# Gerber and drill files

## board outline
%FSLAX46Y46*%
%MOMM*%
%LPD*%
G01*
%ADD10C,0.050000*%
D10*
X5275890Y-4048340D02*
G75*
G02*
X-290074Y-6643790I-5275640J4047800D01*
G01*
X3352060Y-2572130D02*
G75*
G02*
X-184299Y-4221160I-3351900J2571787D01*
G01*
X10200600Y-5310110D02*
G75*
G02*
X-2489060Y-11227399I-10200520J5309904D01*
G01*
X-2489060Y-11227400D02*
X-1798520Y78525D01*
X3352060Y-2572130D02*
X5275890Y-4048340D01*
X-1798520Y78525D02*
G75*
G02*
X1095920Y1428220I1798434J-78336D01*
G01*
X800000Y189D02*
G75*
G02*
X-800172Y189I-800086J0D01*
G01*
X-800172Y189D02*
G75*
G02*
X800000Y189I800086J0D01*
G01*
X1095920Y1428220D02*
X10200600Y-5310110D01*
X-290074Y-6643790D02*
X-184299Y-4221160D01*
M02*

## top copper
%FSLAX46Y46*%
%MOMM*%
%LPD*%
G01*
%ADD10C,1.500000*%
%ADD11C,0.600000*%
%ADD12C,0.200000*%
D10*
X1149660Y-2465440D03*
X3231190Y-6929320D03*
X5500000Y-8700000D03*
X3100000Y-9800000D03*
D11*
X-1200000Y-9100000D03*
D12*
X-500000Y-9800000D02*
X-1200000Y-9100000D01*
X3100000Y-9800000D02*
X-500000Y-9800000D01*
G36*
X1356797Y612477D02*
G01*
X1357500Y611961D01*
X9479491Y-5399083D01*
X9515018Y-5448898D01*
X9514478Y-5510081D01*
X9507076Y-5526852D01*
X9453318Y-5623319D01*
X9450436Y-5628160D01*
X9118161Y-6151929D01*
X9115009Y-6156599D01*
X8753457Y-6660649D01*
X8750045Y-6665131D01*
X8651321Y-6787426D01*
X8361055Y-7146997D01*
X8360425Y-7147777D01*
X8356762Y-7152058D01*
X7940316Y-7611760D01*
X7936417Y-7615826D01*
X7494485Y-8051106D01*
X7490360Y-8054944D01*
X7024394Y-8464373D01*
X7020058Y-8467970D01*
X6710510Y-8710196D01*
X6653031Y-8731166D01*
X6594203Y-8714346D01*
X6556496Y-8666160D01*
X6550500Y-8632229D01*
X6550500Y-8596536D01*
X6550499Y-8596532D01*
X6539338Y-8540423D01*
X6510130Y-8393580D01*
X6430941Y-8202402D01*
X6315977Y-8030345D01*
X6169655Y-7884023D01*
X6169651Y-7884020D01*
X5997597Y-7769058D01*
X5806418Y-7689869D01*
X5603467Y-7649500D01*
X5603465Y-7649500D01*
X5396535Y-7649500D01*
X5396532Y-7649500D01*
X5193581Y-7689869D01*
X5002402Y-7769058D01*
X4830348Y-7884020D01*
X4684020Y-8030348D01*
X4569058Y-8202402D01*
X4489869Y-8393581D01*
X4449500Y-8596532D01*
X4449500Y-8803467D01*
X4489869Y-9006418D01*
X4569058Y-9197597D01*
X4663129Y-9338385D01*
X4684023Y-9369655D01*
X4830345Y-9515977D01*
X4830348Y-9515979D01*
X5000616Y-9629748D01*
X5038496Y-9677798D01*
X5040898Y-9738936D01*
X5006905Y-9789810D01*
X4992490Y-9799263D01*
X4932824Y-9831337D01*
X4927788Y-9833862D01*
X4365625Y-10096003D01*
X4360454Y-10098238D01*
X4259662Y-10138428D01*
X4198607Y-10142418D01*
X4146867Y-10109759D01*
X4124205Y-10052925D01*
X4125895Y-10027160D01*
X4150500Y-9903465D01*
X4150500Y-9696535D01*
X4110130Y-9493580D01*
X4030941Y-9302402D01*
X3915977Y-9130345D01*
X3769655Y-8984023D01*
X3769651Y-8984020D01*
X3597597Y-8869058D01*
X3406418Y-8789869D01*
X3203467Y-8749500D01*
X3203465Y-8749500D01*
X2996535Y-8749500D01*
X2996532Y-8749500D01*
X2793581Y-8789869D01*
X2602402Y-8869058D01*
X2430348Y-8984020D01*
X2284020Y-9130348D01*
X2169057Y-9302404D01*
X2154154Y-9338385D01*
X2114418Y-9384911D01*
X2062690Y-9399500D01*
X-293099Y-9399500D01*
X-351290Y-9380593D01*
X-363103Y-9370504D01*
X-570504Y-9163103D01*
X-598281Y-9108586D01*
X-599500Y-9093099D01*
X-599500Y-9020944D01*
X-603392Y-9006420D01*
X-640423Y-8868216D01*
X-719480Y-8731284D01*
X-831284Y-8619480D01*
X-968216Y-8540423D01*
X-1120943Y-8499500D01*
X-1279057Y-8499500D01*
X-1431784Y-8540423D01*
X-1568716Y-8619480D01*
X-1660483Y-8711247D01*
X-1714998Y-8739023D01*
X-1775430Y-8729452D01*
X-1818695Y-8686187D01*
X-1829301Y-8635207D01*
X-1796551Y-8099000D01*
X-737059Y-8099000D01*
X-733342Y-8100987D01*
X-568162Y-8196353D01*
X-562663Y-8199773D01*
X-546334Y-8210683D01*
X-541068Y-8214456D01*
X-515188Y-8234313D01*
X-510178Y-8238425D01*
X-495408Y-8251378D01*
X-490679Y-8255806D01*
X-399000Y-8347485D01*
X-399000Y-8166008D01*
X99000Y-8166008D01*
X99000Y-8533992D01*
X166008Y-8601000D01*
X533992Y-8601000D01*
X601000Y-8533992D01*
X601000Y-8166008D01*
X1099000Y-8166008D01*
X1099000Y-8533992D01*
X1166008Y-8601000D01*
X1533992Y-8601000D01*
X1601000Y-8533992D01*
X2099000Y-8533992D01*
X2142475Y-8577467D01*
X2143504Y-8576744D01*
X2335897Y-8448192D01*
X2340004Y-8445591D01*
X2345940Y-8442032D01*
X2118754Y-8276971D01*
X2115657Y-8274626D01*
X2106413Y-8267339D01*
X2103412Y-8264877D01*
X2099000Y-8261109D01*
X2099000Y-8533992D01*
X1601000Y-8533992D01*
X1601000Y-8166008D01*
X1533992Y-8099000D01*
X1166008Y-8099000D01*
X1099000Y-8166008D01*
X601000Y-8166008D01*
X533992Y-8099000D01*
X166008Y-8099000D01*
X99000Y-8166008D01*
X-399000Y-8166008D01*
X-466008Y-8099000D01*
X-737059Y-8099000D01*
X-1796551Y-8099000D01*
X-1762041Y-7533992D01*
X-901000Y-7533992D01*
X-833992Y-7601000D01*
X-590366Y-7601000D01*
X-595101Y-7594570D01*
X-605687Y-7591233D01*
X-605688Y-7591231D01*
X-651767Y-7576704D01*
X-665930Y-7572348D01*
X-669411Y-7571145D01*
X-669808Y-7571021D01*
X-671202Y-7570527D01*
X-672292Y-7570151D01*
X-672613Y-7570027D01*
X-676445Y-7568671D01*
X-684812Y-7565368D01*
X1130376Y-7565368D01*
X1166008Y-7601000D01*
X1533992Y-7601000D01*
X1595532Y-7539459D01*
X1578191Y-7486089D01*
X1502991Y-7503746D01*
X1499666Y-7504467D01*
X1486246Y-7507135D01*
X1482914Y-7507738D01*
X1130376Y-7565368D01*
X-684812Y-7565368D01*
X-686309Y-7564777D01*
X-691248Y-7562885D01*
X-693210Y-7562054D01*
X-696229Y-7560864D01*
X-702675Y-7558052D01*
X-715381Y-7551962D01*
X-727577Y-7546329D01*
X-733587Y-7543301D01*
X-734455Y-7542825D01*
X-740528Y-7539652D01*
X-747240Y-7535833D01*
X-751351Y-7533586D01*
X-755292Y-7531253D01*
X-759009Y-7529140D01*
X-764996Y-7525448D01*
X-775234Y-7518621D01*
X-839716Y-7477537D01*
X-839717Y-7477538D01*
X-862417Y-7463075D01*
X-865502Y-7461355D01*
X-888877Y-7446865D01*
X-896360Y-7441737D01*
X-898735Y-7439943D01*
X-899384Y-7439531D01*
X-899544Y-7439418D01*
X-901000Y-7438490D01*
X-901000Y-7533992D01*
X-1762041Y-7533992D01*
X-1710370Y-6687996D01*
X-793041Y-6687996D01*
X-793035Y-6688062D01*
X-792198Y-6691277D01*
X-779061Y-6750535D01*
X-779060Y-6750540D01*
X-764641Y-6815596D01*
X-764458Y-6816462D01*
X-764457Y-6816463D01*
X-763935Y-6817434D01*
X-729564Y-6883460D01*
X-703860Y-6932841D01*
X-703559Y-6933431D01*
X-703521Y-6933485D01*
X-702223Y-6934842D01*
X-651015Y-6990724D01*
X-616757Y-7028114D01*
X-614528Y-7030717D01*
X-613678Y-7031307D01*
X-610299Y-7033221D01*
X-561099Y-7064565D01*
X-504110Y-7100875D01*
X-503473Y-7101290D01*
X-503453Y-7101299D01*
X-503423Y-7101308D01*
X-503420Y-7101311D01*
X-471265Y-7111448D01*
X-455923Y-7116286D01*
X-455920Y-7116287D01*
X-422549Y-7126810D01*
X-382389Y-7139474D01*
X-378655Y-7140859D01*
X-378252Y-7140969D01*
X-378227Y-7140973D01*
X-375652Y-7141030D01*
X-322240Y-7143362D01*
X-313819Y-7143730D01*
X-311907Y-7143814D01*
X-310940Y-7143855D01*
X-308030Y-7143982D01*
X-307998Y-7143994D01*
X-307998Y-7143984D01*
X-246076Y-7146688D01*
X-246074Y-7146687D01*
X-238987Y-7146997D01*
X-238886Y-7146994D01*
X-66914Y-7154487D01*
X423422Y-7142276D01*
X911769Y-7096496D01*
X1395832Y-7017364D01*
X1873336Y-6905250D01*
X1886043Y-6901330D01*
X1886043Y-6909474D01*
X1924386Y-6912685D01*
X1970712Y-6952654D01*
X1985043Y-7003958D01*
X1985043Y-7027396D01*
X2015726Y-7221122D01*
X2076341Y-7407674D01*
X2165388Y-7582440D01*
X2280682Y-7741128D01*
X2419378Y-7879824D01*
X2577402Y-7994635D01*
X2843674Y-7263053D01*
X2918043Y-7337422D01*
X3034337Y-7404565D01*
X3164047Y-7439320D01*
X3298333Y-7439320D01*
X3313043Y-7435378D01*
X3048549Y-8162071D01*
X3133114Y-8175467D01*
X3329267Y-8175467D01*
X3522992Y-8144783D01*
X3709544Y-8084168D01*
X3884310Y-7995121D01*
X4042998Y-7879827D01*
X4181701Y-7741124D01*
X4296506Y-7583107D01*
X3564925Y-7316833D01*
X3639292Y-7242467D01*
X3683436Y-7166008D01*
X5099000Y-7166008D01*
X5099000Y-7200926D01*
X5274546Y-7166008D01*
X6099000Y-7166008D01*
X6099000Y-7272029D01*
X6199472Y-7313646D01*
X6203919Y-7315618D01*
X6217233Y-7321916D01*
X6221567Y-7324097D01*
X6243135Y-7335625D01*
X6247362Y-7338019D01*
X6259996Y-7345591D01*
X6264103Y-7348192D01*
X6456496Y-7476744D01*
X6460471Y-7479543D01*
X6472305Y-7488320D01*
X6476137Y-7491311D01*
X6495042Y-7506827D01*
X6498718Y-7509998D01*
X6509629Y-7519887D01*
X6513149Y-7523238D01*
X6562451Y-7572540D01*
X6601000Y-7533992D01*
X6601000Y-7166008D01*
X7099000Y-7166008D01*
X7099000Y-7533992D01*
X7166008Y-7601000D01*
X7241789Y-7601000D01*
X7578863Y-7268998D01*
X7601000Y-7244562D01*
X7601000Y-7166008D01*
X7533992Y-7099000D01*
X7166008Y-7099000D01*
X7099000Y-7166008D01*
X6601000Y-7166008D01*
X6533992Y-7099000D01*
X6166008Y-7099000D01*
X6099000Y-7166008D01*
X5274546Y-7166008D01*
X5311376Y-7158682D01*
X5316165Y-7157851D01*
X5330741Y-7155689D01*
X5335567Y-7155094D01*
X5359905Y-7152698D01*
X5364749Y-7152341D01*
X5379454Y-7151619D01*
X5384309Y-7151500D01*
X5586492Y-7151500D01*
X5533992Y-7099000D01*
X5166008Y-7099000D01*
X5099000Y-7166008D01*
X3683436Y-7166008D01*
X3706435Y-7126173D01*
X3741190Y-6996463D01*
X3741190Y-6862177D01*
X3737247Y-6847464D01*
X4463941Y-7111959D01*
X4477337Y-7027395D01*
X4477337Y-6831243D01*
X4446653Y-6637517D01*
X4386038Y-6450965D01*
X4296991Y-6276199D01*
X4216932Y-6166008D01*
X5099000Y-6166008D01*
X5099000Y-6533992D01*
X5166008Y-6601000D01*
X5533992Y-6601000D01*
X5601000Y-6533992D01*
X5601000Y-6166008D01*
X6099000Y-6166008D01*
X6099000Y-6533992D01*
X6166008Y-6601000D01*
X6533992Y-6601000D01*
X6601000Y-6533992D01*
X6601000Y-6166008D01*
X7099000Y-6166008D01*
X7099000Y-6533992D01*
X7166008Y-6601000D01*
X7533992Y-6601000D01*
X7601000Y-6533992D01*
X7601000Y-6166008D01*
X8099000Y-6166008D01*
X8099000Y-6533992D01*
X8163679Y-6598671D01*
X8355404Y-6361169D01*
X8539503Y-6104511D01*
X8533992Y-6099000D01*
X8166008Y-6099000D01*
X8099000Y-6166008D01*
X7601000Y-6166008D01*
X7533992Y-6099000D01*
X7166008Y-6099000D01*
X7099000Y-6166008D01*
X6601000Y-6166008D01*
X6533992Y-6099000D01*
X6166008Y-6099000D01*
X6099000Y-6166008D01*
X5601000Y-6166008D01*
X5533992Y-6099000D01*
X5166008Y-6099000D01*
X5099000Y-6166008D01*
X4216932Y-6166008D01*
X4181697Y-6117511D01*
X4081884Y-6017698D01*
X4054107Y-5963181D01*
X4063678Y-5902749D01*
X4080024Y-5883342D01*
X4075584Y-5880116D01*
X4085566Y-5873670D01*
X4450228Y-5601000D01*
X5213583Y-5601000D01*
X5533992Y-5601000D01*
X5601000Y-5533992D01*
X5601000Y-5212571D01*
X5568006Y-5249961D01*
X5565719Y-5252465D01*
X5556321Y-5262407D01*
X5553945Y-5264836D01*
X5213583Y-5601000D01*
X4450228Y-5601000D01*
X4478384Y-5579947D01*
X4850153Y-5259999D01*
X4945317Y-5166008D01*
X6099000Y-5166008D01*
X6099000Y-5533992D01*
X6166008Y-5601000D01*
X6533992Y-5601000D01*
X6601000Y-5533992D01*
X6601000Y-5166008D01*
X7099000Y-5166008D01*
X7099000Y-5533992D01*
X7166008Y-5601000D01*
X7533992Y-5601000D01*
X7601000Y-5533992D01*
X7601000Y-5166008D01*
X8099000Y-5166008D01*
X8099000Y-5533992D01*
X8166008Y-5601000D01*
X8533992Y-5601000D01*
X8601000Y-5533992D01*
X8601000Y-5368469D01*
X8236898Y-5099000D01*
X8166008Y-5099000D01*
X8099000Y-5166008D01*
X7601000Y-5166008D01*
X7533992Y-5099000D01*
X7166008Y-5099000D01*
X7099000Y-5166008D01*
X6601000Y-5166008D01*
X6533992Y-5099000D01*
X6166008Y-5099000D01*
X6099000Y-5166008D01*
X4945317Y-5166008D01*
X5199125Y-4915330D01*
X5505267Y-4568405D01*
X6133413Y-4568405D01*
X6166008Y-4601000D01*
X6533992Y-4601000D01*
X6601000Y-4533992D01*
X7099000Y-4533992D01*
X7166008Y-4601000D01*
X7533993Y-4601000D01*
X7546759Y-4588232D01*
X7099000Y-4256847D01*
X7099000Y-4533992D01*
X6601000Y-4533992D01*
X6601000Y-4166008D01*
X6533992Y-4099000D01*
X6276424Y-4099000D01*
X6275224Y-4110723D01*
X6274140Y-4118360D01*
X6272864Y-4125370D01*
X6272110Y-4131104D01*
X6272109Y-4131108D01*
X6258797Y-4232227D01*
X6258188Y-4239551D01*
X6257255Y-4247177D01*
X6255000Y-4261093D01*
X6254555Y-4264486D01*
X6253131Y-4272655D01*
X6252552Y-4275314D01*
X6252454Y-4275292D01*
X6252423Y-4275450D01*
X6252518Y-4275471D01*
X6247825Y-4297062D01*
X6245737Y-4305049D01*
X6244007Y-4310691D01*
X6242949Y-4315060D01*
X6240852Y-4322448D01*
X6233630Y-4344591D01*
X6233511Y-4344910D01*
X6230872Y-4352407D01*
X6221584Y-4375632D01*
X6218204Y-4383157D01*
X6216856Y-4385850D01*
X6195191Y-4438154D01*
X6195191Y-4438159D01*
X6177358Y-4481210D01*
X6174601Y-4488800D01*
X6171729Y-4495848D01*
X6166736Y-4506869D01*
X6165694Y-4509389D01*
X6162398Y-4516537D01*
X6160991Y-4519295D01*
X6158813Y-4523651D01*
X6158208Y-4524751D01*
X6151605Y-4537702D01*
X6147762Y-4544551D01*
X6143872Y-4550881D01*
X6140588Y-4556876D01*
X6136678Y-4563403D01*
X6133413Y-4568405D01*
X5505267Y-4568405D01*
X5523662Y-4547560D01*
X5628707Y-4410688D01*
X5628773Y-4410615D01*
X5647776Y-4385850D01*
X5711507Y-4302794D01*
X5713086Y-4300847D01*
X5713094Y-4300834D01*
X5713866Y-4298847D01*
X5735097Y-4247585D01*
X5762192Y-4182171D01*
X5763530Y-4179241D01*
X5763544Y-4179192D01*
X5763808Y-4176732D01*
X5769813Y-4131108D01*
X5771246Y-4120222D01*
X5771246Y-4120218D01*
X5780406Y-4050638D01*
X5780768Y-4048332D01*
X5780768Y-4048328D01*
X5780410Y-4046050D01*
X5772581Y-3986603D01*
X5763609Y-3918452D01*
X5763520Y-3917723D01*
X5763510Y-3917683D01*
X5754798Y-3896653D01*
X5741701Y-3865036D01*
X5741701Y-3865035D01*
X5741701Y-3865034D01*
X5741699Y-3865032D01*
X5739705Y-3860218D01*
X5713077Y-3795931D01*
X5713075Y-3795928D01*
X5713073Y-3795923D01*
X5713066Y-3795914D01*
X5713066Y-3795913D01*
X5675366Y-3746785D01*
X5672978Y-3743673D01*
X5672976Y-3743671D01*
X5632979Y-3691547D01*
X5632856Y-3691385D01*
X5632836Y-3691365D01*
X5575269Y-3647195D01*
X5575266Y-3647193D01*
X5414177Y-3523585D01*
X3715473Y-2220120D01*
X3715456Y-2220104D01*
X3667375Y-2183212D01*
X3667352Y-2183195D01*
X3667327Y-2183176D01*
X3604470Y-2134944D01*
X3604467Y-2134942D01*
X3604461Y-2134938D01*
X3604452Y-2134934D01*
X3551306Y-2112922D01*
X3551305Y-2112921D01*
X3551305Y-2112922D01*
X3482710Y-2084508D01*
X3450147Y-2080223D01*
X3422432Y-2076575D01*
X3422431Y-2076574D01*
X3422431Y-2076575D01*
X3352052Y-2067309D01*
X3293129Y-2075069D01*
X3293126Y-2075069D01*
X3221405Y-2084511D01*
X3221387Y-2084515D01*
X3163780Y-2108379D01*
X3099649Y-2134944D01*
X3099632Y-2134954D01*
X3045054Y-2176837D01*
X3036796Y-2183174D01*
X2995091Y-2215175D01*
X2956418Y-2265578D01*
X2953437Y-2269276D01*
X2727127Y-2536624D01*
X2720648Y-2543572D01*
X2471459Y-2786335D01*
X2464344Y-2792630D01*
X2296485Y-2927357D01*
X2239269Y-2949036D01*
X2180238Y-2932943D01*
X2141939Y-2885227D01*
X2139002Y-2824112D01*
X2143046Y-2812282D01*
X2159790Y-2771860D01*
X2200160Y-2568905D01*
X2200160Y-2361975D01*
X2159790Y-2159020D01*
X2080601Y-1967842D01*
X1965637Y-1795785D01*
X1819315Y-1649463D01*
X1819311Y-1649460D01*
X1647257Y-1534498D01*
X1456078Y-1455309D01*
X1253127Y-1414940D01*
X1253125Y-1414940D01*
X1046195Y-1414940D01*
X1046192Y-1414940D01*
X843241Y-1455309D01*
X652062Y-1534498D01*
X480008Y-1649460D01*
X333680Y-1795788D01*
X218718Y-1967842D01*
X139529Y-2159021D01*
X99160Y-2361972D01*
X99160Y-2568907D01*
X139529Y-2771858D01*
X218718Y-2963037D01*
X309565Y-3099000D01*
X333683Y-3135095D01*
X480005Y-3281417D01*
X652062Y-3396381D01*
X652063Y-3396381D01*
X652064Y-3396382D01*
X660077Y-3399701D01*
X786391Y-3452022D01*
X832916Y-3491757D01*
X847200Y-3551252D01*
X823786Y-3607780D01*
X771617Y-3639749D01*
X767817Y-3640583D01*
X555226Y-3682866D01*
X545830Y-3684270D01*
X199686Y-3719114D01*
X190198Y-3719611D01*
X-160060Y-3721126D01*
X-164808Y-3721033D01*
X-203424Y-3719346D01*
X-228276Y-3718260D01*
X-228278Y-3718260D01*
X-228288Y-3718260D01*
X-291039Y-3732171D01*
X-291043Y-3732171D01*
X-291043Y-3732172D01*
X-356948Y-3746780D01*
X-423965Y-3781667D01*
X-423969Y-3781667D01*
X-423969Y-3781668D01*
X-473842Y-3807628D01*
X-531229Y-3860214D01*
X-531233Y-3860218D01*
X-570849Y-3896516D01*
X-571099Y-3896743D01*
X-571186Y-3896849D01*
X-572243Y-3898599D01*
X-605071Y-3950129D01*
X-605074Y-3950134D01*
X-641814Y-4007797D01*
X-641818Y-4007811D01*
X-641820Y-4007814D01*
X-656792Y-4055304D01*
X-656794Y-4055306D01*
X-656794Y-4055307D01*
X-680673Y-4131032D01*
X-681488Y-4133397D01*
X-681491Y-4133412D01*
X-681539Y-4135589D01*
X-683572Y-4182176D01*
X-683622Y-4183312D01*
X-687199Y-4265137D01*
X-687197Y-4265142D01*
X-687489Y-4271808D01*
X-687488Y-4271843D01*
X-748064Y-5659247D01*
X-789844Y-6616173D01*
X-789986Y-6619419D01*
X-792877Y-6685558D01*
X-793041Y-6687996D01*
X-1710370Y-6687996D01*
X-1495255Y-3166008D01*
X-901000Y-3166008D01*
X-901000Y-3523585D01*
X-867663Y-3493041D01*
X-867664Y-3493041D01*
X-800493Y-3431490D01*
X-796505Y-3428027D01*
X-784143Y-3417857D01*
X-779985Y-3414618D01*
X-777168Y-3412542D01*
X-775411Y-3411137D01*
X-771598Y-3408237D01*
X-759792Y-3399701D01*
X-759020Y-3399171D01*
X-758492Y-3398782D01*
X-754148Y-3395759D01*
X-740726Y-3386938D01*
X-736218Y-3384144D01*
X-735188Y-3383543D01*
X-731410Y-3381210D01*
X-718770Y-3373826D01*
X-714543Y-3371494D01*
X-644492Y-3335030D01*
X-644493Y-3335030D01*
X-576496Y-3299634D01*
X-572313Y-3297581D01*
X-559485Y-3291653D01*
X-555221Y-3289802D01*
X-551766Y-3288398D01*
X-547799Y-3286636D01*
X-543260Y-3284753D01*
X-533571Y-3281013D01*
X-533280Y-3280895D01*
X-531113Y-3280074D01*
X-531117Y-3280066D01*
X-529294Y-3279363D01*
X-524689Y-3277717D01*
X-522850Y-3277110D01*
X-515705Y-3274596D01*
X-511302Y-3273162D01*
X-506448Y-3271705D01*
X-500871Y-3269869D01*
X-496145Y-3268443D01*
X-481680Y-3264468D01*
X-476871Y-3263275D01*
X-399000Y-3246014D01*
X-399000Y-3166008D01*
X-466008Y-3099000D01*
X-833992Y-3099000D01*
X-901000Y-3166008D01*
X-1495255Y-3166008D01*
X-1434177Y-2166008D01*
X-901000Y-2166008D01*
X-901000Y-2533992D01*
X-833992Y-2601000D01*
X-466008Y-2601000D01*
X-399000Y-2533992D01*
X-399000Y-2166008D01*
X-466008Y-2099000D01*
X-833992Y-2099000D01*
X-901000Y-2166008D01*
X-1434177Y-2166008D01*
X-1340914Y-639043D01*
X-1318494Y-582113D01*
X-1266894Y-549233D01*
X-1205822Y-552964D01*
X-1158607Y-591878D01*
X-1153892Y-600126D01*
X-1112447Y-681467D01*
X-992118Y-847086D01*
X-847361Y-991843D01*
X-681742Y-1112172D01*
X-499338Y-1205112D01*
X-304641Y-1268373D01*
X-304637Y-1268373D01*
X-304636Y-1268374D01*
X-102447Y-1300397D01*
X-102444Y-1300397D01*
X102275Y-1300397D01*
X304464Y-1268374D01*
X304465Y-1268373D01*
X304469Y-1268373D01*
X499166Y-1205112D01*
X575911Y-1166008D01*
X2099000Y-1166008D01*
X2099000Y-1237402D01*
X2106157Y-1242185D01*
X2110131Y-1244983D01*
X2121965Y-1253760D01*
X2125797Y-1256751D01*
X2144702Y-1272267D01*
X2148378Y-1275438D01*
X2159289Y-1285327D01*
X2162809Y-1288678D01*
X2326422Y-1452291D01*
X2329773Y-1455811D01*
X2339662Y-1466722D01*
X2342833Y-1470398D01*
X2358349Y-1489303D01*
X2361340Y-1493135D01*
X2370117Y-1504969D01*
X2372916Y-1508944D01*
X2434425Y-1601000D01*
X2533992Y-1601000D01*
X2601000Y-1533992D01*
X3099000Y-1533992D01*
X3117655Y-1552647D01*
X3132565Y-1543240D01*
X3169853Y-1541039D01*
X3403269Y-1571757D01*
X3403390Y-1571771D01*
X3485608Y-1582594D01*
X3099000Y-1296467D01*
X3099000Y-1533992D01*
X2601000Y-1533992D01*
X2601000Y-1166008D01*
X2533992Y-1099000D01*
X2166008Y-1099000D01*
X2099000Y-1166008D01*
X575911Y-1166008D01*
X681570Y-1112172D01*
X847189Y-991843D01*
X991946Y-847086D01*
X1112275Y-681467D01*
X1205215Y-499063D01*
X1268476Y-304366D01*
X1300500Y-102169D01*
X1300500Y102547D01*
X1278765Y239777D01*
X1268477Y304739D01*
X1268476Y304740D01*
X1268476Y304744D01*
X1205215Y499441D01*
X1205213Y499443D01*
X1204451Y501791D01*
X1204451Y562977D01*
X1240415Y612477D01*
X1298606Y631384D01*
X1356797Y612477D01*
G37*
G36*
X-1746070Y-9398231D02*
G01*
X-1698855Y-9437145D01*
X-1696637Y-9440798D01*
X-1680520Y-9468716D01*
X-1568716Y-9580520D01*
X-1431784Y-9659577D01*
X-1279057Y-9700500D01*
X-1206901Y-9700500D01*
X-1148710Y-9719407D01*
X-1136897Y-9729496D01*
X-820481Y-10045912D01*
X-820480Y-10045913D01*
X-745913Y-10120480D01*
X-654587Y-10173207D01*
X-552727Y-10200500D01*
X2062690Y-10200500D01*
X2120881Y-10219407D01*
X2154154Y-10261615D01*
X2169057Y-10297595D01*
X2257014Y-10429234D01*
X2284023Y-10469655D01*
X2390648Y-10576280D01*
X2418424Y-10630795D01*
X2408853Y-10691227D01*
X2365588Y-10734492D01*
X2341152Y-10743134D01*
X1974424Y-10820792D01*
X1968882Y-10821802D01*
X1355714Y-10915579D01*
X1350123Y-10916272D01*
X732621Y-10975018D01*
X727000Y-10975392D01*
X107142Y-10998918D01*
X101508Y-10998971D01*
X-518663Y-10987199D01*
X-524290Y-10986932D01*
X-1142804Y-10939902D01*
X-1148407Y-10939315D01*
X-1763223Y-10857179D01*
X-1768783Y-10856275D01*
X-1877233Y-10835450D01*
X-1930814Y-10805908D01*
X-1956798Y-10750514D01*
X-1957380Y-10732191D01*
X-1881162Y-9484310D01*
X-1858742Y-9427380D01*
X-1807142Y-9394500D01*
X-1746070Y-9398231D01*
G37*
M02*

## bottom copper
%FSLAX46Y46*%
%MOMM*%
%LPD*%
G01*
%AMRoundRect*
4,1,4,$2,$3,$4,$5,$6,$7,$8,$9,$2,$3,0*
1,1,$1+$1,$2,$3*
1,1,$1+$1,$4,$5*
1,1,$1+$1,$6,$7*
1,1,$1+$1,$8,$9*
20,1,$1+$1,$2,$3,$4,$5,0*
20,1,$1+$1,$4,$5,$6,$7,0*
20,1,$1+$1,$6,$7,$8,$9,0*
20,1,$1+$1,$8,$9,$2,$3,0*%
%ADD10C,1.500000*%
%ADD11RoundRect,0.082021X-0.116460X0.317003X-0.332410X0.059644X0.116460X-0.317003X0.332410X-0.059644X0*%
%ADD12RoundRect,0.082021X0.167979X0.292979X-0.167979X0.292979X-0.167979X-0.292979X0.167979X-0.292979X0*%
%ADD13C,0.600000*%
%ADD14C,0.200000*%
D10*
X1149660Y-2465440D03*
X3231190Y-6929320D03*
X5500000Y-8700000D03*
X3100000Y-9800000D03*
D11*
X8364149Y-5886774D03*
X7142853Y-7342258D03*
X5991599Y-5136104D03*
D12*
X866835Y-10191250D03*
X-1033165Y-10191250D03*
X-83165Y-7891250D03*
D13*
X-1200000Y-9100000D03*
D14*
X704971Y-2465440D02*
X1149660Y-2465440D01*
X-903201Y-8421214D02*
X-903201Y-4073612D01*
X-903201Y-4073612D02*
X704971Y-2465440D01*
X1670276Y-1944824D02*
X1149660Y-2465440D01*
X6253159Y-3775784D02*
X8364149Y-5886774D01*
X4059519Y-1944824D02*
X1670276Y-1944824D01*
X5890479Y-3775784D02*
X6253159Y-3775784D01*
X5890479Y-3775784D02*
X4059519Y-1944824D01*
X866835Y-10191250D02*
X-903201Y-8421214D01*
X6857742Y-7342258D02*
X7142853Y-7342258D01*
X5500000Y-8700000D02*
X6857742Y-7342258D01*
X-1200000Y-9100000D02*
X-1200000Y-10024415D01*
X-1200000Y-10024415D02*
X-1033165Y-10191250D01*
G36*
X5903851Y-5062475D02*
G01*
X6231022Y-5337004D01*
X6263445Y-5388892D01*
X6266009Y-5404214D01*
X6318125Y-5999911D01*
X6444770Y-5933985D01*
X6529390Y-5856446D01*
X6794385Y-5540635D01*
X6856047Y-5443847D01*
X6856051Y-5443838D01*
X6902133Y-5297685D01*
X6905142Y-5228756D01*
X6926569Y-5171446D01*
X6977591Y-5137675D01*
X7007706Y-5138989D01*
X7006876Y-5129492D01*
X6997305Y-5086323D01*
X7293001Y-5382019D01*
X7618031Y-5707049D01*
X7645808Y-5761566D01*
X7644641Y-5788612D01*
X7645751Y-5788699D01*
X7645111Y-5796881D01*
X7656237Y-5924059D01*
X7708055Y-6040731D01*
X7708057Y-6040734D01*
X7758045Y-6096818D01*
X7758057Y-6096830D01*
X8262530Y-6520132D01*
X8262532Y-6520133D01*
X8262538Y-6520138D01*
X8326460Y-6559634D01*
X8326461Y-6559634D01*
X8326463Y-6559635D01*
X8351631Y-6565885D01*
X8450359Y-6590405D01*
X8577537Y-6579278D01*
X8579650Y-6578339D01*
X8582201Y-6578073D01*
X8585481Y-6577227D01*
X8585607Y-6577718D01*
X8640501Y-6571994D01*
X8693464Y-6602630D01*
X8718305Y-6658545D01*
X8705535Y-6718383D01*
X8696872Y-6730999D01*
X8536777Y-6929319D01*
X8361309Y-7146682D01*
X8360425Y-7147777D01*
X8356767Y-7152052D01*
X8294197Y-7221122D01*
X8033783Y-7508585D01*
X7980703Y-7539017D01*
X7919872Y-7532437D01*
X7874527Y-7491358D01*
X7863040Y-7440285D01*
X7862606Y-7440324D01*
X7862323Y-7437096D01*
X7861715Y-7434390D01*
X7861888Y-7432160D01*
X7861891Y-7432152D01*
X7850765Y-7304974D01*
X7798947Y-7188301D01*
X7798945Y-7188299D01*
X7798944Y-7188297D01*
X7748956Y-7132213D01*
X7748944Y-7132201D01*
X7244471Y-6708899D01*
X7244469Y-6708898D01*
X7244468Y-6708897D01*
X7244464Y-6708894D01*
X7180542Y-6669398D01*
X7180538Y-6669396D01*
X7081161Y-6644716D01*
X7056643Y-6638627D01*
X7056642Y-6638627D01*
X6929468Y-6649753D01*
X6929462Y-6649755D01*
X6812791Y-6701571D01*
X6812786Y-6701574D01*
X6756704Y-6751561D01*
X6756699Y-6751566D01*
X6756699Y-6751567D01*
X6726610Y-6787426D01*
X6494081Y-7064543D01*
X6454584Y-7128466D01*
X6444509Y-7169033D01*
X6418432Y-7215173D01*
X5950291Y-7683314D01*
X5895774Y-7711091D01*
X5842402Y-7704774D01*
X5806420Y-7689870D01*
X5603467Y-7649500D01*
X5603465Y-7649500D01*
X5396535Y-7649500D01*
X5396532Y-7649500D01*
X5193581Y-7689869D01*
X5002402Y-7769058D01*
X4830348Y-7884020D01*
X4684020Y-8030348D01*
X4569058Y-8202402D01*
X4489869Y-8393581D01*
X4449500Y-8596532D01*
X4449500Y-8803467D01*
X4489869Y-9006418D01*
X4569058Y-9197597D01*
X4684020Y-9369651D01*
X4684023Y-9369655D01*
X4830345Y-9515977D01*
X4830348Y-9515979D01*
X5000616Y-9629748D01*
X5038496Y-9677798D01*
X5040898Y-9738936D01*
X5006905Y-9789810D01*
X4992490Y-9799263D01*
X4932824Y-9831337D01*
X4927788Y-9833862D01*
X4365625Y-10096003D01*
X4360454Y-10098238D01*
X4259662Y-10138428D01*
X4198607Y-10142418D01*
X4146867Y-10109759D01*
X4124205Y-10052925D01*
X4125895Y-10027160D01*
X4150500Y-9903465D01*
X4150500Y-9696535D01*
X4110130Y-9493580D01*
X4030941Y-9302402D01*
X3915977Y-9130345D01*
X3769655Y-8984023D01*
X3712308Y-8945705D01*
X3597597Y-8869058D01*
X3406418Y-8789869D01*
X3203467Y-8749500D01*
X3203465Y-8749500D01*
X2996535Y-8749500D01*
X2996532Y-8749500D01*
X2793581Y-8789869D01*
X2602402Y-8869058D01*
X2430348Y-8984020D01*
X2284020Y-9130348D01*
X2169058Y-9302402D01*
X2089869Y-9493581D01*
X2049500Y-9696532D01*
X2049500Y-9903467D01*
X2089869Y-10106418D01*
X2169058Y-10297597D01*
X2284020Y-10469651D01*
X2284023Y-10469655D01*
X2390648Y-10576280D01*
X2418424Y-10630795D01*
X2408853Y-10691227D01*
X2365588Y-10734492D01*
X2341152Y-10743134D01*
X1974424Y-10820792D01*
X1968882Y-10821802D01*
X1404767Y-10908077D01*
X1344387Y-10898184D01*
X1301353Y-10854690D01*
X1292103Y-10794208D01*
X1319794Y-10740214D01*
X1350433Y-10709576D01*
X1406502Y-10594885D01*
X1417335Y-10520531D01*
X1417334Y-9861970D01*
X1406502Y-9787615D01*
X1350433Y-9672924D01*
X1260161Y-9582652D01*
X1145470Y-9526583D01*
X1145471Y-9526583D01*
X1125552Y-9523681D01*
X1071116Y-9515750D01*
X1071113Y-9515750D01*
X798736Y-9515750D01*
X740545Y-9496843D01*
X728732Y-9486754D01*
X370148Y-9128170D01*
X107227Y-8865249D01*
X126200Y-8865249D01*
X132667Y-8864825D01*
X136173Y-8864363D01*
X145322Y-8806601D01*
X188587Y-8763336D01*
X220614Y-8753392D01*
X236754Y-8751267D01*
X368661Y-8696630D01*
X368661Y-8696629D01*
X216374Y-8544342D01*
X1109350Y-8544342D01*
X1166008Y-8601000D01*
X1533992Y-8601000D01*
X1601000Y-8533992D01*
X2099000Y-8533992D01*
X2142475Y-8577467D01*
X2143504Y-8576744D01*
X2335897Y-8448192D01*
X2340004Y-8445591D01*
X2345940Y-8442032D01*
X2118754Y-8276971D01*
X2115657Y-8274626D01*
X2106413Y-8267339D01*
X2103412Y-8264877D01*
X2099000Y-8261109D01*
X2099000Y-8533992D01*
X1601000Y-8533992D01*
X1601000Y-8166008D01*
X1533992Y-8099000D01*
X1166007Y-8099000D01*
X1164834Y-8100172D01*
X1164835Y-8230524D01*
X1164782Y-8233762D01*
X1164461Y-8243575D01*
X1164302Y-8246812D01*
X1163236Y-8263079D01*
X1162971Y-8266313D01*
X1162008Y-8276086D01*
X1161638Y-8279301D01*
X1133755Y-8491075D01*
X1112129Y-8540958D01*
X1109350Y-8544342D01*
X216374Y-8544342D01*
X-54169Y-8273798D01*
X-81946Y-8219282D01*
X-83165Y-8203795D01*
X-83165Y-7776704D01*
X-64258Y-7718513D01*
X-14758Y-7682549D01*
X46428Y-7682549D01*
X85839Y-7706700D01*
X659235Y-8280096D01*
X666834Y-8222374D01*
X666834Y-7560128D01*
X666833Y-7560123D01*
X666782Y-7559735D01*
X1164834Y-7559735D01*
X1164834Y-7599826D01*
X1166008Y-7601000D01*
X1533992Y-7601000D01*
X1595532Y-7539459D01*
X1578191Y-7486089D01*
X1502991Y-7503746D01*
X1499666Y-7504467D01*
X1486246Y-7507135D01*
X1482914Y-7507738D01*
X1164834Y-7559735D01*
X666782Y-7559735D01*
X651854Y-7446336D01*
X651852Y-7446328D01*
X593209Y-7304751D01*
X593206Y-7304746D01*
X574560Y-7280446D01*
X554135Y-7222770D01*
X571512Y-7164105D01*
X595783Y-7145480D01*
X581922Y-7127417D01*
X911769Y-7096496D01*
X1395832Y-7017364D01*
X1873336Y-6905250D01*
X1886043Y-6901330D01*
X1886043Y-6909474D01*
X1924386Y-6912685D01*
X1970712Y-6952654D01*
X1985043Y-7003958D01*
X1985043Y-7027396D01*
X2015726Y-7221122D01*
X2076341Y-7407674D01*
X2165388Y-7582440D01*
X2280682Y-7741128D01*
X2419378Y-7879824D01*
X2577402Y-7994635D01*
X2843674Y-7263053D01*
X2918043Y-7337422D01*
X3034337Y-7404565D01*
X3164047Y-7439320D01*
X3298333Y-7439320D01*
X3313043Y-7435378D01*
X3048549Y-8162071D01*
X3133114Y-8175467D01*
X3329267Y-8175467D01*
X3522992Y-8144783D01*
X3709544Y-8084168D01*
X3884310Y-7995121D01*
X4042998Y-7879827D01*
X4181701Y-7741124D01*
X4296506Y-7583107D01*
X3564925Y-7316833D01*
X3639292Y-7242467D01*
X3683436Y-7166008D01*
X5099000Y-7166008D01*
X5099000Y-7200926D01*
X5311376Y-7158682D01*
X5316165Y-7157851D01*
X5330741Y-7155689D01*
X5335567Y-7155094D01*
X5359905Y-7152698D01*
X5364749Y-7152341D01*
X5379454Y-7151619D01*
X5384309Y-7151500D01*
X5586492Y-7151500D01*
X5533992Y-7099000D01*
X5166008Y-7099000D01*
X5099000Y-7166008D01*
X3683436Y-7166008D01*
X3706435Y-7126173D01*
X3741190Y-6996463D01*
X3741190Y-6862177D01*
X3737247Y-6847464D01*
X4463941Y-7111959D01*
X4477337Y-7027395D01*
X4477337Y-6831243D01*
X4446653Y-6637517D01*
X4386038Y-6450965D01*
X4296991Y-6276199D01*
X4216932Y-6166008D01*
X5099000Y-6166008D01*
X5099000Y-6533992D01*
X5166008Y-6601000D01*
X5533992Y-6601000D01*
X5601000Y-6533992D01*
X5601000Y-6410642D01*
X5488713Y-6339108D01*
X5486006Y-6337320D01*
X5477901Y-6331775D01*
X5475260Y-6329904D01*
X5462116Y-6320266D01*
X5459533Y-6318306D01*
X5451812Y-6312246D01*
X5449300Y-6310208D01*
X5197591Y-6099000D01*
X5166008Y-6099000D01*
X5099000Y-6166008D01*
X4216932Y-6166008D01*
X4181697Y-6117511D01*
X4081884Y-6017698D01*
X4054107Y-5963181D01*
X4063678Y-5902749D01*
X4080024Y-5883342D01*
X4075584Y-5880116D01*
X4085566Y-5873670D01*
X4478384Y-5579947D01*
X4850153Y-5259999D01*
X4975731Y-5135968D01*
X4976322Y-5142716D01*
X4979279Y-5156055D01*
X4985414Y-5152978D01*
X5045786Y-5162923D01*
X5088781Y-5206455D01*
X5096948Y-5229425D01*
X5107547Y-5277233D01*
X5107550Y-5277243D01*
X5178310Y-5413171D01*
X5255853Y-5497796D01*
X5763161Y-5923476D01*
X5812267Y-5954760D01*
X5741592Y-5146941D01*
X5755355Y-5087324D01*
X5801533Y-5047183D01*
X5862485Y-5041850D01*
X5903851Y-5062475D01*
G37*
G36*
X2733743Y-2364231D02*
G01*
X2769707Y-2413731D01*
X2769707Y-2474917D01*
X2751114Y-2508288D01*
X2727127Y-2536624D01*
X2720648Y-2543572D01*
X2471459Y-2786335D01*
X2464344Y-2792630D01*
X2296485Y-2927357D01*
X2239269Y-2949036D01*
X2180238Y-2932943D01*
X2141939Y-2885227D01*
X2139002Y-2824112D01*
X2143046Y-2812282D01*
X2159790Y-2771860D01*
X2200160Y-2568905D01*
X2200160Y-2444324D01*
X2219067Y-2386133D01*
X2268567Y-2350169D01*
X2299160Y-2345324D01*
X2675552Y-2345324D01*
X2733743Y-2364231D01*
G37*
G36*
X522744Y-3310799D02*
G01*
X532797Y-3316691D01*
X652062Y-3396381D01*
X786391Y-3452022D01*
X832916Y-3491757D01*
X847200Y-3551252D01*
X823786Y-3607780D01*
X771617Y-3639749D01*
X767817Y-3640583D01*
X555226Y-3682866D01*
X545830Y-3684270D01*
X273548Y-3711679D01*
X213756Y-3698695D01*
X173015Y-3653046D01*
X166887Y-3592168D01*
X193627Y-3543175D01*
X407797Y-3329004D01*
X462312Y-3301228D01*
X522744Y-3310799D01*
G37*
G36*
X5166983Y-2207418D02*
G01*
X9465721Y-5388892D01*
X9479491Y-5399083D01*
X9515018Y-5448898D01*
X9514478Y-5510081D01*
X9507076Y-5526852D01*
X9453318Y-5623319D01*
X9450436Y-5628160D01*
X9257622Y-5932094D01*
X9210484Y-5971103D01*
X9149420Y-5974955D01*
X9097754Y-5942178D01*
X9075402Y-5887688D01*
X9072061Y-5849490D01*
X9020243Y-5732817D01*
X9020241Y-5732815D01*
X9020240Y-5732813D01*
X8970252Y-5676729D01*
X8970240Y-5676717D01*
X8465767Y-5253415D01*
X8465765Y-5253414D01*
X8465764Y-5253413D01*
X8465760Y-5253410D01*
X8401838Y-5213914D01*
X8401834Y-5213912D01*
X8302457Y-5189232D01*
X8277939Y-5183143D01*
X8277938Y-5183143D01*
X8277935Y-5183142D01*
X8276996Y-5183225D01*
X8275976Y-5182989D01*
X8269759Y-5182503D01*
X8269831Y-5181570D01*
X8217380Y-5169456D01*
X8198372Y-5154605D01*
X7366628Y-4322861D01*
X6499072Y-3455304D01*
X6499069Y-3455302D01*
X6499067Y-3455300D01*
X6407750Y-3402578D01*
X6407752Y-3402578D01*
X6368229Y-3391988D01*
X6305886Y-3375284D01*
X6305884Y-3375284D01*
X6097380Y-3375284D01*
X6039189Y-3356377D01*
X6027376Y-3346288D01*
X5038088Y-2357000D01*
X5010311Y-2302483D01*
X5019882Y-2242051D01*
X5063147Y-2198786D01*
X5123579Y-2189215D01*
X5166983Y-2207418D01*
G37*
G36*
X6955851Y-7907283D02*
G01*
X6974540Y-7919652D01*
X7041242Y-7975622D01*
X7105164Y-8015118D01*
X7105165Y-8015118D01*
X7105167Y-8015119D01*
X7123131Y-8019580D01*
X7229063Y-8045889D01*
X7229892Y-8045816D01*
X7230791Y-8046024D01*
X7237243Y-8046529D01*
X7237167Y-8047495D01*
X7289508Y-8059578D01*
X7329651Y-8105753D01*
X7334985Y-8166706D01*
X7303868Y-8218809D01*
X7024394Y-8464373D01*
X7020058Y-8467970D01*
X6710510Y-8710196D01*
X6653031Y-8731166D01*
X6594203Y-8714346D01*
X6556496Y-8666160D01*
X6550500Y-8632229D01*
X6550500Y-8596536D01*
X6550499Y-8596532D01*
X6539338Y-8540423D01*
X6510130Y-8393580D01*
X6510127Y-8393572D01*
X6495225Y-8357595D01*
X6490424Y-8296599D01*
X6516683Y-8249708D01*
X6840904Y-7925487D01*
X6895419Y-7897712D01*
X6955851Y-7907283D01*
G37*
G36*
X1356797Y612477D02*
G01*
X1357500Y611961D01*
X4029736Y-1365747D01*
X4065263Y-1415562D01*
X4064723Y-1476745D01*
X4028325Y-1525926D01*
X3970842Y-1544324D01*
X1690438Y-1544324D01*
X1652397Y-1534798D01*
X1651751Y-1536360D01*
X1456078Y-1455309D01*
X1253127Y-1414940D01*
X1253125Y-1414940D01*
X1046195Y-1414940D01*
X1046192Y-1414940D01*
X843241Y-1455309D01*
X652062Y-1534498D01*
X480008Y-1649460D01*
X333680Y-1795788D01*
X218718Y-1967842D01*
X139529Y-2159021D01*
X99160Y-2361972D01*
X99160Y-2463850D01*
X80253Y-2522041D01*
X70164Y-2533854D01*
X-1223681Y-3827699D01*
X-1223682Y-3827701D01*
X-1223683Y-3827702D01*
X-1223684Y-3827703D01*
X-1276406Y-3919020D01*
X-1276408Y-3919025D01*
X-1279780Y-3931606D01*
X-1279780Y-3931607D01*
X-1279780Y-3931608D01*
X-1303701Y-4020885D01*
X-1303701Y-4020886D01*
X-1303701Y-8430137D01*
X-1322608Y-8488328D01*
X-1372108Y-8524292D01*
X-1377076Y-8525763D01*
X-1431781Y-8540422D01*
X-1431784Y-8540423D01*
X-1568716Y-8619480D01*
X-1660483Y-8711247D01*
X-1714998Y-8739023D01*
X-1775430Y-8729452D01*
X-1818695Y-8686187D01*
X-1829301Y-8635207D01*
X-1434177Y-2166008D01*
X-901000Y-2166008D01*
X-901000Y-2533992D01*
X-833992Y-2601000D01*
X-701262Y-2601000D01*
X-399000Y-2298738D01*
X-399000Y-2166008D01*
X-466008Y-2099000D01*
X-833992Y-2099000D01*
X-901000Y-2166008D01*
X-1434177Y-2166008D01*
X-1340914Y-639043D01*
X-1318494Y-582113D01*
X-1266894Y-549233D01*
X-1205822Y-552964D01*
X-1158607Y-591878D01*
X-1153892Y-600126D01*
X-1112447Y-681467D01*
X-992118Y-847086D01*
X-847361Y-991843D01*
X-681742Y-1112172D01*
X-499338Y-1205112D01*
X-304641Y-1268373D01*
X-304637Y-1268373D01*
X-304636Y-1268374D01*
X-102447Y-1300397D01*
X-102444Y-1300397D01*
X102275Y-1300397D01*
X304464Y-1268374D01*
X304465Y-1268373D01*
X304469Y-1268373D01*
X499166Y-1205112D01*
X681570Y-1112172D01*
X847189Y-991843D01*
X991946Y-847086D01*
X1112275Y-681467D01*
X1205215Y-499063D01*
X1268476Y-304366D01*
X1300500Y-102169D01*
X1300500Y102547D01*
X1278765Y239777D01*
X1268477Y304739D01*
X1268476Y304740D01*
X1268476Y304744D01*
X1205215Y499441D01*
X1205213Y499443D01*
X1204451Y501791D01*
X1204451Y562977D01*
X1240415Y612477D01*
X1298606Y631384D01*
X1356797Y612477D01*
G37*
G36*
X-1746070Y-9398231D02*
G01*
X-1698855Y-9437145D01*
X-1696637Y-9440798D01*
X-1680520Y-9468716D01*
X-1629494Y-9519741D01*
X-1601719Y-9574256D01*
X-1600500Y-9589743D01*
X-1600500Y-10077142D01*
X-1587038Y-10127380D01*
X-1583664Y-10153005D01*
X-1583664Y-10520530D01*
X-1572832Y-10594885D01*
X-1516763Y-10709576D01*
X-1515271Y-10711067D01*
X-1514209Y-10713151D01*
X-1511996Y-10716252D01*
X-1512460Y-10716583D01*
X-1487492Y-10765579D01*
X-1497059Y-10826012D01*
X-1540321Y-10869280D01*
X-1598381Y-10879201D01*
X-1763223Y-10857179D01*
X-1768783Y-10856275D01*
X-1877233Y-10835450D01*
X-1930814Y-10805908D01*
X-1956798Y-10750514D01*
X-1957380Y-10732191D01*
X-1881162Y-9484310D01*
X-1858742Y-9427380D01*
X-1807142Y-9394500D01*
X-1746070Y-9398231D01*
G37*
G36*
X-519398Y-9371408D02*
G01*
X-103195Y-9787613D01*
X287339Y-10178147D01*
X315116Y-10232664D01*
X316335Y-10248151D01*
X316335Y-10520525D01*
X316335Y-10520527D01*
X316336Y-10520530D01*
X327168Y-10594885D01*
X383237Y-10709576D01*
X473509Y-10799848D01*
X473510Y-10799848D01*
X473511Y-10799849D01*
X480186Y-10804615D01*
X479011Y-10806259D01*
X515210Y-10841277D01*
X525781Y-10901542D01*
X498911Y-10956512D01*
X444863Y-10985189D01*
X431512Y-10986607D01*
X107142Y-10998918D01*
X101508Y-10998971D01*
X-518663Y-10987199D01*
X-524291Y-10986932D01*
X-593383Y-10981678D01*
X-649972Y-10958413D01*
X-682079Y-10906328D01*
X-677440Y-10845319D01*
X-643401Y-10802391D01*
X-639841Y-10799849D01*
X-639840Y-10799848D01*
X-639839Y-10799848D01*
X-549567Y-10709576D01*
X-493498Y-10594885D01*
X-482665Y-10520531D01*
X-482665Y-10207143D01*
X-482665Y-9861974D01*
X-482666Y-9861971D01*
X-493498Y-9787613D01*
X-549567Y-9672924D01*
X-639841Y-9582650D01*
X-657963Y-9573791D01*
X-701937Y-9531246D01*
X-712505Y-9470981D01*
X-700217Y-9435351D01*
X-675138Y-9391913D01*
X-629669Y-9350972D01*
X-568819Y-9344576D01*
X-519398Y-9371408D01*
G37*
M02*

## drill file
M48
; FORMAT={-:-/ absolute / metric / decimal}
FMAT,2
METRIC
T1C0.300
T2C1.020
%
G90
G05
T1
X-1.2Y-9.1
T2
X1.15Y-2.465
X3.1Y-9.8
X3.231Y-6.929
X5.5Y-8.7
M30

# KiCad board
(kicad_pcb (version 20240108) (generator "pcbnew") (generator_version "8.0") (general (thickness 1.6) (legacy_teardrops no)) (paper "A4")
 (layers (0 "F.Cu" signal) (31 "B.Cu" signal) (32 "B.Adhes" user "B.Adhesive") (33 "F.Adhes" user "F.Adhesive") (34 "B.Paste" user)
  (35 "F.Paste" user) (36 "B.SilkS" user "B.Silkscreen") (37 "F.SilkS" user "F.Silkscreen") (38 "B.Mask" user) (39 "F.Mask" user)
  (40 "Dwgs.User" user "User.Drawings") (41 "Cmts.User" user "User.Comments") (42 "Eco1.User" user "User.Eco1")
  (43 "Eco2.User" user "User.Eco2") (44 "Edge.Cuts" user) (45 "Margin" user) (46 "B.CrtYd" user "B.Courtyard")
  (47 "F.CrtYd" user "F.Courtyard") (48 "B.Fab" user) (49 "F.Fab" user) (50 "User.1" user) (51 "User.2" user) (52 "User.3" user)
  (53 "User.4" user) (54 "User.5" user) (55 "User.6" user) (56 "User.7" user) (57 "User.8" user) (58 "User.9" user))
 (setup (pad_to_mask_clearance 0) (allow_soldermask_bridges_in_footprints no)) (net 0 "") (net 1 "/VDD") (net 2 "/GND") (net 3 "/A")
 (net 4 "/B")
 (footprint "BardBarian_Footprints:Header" (layer "F.Cu") (at 1.14966 2.46544 25)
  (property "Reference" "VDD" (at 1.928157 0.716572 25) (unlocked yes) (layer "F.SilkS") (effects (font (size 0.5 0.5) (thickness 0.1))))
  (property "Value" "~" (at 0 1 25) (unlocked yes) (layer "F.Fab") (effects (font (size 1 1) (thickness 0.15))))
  (pad "1" thru_hole circle (at 0 0 25) (size 1.5 1.5) (drill 1.02) (layers "*.Cu" "*.Mask") (remove_unused_layers no) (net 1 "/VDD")))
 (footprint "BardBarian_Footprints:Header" (layer "F.Cu") (at 3.23119 6.92932 25)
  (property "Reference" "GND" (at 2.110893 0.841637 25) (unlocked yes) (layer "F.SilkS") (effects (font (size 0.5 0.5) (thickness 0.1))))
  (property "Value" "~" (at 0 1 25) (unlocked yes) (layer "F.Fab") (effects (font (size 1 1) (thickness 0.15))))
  (pad "1" thru_hole circle (at 0 0 25) (size 1.5 1.5) (drill 1.02) (layers "*.Cu" "*.Mask") (remove_unused_layers no) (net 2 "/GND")))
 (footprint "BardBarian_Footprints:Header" (layer "F.Cu") (at 5.5 8.7 25)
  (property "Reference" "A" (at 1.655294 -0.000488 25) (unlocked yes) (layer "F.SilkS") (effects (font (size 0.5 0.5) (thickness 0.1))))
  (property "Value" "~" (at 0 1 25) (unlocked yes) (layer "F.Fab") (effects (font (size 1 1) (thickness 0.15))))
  (pad "1" thru_hole circle (at 0 0 25) (size 1.5 1.5) (drill 1.02) (layers "*.Cu" "*.Mask") (remove_unused_layers no) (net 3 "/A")))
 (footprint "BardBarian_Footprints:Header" (layer "F.Cu") (at 3.1 9.8 25)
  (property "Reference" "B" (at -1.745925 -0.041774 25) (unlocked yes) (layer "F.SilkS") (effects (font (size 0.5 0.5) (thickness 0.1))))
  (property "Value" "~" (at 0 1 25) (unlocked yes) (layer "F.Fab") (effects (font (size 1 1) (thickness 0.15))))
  (pad "1" thru_hole circle (at 0 0 25) (size 1.5 1.5) (drill 1.02) (layers "*.Cu" "*.Mask") (remove_unused_layers no) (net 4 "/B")))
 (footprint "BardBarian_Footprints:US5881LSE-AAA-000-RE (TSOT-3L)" (layer "B.Cu") (at 6.87255 5.87531 -130)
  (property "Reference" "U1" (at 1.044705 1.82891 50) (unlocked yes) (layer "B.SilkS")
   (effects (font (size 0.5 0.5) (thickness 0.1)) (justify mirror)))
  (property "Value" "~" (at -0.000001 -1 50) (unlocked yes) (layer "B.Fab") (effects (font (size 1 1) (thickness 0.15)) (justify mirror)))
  (pad "1" smd roundrect (at -0.949999 -1.15 230) (size 0.5 0.75) (layers "B.Cu" "B.Paste" "B.Mask") (roundrect_rratio 0.1640419948)
   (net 1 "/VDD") (thermal_bridge_angle 45))
  (pad "2" smd roundrect (at 0.95 -1.15 230) (size 0.5 0.75) (layers "B.Cu" "B.Paste" "B.Mask") (roundrect_rratio 0.1640419948) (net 3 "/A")
   (thermal_bridge_angle 45))
  (pad "3" smd roundrect (at 0 1.15 230) (size 0.5 0.75) (layers "B.Cu" "B.Paste" "B.Mask") (roundrect_rratio 0.1640419948) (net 2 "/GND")
   (thermal_bridge_angle 45)))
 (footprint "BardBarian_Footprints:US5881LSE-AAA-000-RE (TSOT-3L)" (layer "B.Cu") (at -0.083165 9.04125 180)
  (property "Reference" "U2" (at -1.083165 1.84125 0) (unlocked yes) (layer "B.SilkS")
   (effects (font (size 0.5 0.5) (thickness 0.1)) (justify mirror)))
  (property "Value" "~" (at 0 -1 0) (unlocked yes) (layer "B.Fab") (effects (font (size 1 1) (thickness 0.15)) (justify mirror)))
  (pad "1" smd roundrect (at -0.95 -1.15 180) (size 0.5 0.75) (layers "B.Cu" "B.Paste" "B.Mask") (roundrect_rratio 0.1640419948)
   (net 1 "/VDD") (thermal_bridge_angle 45))
  (pad "2" smd roundrect (at 0.95 -1.15 180) (size 0.5 0.75) (layers "B.Cu" "B.Paste" "B.Mask") (roundrect_rratio 0.1640419948) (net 4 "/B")
   (thermal_bridge_angle 45))
  (pad "3" smd roundrect (at 0 1.15 180) (size 0.5 0.75) (layers "B.Cu" "B.Paste" "B.Mask") (roundrect_rratio 0.1640419948) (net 2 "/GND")
   (thermal_bridge_angle 45)))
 (gr_arc (start 5.27589 4.04834) (mid 2.810487 6.027117) (end -0.290074 6.64379) (stroke (width 0.05) (type default)) (layer "Edge.Cuts"))
 (gr_arc (start 3.35206 2.57213) (mid 1.785656 3.829354) (end -0.184299 4.22116) (stroke (width 0.05) (type default)) (layer "Edge.Cuts"))
 (gr_arc (start 10.2006 5.31011) (mid 4.860113 10.422575) (end -2.48906 11.2274) (stroke (width 0.05) (type default)) (layer "Edge.Cuts"))
 (gr_line (start -2.48906 11.2274) (end -1.79852 -0.078525) (stroke (width 0.05) (type default)) (layer "Edge.Cuts"))
 (gr_line (start 3.35206 2.57213) (end 5.27589 4.04834) (stroke (width 0.05) (type default)) (layer "Edge.Cuts"))
 (gr_arc (start -1.79852 -0.078525) (mid -0.760856 -1.63167) (end 1.09592 -1.42822) (stroke (width 0.05) (type default)) (layer "Edge.Cuts"))
 (gr_circle (center -0.000086 -0.000189) (end 0.8 0) (stroke (width 0.05) (type default)) (fill none) (layer "Edge.Cuts"))
 (gr_line (start 1.09592 -1.42822) (end 10.2006 5.31011) (stroke (width 0.05) (type default)) (layer "Edge.Cuts"))
 (gr_line (start -0.290074 6.64379) (end -0.184299 4.22116) (stroke (width 0.05) (type default)) (layer "Edge.Cuts"))
 (segment (start 0.704971 2.46544) (end 1.14966 2.46544) (width 0.2) (layer "B.Cu") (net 1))
 (segment (start -0.903201 8.421214) (end -0.903201 4.073612) (width 0.2) (layer "B.Cu") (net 1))
 (segment (start -0.903201 4.073612) (end 0.704971 2.46544) (width 0.2) (layer "B.Cu") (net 1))
 (segment (start 1.670276 1.944824) (end 1.14966 2.46544) (width 0.2) (layer "B.Cu") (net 1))
 (segment (start 6.253159 3.775784) (end 8.364149 5.886774) (width 0.2) (layer "B.Cu") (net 1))
 (segment (start 4.059519 1.944824) (end 1.670276 1.944824) (width 0.2) (layer "B.Cu") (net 1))
 (segment (start 5.890479 3.775784) (end 6.253159 3.775784) (width 0.2) (layer "B.Cu") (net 1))
 (segment (start 5.890479 3.775784) (end 4.059519 1.944824) (width 0.2) (layer "B.Cu") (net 1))
 (segment (start 0.866835 10.19125) (end -0.903201 8.421214) (width 0.2) (layer "B.Cu") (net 1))
 (segment (start 6.857742 7.342258) (end 7.142853 7.342258) (width 0.2) (layer "B.Cu") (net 3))
 (segment (start 5.5 8.7) (end 6.857742 7.342258) (width 0.2) (layer "B.Cu") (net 3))
 (segment (start -0.5 9.8) (end -1.2 9.1) (width 0.2) (layer "F.Cu") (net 4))
 (segment (start 3.1 9.8) (end -0.5 9.8) (width 0.2) (layer "F.Cu") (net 4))
 (via (at -1.2 9.1) (size 0.6) (drill 0.3) (layers "F.Cu" "B.Cu") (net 4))
 (segment (start -1.2 9.1) (end -1.2 10.024415) (width 0.2) (layer "B.Cu") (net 4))
 (segment (start -1.2 10.024415) (end -1.033165 10.19125) (width 0.2) (layer "B.Cu") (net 4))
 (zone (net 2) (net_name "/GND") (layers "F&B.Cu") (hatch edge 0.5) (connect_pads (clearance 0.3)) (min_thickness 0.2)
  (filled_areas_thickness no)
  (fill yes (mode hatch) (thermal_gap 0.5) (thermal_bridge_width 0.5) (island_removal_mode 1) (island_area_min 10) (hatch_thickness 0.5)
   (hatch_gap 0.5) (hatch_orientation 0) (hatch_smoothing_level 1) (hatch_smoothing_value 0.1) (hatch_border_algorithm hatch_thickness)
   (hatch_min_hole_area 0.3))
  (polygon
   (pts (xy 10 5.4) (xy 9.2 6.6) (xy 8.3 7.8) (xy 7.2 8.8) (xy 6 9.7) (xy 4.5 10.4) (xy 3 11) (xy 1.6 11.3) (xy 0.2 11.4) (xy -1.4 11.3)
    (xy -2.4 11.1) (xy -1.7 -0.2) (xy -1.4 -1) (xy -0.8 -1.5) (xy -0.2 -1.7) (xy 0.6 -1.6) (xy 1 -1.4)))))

